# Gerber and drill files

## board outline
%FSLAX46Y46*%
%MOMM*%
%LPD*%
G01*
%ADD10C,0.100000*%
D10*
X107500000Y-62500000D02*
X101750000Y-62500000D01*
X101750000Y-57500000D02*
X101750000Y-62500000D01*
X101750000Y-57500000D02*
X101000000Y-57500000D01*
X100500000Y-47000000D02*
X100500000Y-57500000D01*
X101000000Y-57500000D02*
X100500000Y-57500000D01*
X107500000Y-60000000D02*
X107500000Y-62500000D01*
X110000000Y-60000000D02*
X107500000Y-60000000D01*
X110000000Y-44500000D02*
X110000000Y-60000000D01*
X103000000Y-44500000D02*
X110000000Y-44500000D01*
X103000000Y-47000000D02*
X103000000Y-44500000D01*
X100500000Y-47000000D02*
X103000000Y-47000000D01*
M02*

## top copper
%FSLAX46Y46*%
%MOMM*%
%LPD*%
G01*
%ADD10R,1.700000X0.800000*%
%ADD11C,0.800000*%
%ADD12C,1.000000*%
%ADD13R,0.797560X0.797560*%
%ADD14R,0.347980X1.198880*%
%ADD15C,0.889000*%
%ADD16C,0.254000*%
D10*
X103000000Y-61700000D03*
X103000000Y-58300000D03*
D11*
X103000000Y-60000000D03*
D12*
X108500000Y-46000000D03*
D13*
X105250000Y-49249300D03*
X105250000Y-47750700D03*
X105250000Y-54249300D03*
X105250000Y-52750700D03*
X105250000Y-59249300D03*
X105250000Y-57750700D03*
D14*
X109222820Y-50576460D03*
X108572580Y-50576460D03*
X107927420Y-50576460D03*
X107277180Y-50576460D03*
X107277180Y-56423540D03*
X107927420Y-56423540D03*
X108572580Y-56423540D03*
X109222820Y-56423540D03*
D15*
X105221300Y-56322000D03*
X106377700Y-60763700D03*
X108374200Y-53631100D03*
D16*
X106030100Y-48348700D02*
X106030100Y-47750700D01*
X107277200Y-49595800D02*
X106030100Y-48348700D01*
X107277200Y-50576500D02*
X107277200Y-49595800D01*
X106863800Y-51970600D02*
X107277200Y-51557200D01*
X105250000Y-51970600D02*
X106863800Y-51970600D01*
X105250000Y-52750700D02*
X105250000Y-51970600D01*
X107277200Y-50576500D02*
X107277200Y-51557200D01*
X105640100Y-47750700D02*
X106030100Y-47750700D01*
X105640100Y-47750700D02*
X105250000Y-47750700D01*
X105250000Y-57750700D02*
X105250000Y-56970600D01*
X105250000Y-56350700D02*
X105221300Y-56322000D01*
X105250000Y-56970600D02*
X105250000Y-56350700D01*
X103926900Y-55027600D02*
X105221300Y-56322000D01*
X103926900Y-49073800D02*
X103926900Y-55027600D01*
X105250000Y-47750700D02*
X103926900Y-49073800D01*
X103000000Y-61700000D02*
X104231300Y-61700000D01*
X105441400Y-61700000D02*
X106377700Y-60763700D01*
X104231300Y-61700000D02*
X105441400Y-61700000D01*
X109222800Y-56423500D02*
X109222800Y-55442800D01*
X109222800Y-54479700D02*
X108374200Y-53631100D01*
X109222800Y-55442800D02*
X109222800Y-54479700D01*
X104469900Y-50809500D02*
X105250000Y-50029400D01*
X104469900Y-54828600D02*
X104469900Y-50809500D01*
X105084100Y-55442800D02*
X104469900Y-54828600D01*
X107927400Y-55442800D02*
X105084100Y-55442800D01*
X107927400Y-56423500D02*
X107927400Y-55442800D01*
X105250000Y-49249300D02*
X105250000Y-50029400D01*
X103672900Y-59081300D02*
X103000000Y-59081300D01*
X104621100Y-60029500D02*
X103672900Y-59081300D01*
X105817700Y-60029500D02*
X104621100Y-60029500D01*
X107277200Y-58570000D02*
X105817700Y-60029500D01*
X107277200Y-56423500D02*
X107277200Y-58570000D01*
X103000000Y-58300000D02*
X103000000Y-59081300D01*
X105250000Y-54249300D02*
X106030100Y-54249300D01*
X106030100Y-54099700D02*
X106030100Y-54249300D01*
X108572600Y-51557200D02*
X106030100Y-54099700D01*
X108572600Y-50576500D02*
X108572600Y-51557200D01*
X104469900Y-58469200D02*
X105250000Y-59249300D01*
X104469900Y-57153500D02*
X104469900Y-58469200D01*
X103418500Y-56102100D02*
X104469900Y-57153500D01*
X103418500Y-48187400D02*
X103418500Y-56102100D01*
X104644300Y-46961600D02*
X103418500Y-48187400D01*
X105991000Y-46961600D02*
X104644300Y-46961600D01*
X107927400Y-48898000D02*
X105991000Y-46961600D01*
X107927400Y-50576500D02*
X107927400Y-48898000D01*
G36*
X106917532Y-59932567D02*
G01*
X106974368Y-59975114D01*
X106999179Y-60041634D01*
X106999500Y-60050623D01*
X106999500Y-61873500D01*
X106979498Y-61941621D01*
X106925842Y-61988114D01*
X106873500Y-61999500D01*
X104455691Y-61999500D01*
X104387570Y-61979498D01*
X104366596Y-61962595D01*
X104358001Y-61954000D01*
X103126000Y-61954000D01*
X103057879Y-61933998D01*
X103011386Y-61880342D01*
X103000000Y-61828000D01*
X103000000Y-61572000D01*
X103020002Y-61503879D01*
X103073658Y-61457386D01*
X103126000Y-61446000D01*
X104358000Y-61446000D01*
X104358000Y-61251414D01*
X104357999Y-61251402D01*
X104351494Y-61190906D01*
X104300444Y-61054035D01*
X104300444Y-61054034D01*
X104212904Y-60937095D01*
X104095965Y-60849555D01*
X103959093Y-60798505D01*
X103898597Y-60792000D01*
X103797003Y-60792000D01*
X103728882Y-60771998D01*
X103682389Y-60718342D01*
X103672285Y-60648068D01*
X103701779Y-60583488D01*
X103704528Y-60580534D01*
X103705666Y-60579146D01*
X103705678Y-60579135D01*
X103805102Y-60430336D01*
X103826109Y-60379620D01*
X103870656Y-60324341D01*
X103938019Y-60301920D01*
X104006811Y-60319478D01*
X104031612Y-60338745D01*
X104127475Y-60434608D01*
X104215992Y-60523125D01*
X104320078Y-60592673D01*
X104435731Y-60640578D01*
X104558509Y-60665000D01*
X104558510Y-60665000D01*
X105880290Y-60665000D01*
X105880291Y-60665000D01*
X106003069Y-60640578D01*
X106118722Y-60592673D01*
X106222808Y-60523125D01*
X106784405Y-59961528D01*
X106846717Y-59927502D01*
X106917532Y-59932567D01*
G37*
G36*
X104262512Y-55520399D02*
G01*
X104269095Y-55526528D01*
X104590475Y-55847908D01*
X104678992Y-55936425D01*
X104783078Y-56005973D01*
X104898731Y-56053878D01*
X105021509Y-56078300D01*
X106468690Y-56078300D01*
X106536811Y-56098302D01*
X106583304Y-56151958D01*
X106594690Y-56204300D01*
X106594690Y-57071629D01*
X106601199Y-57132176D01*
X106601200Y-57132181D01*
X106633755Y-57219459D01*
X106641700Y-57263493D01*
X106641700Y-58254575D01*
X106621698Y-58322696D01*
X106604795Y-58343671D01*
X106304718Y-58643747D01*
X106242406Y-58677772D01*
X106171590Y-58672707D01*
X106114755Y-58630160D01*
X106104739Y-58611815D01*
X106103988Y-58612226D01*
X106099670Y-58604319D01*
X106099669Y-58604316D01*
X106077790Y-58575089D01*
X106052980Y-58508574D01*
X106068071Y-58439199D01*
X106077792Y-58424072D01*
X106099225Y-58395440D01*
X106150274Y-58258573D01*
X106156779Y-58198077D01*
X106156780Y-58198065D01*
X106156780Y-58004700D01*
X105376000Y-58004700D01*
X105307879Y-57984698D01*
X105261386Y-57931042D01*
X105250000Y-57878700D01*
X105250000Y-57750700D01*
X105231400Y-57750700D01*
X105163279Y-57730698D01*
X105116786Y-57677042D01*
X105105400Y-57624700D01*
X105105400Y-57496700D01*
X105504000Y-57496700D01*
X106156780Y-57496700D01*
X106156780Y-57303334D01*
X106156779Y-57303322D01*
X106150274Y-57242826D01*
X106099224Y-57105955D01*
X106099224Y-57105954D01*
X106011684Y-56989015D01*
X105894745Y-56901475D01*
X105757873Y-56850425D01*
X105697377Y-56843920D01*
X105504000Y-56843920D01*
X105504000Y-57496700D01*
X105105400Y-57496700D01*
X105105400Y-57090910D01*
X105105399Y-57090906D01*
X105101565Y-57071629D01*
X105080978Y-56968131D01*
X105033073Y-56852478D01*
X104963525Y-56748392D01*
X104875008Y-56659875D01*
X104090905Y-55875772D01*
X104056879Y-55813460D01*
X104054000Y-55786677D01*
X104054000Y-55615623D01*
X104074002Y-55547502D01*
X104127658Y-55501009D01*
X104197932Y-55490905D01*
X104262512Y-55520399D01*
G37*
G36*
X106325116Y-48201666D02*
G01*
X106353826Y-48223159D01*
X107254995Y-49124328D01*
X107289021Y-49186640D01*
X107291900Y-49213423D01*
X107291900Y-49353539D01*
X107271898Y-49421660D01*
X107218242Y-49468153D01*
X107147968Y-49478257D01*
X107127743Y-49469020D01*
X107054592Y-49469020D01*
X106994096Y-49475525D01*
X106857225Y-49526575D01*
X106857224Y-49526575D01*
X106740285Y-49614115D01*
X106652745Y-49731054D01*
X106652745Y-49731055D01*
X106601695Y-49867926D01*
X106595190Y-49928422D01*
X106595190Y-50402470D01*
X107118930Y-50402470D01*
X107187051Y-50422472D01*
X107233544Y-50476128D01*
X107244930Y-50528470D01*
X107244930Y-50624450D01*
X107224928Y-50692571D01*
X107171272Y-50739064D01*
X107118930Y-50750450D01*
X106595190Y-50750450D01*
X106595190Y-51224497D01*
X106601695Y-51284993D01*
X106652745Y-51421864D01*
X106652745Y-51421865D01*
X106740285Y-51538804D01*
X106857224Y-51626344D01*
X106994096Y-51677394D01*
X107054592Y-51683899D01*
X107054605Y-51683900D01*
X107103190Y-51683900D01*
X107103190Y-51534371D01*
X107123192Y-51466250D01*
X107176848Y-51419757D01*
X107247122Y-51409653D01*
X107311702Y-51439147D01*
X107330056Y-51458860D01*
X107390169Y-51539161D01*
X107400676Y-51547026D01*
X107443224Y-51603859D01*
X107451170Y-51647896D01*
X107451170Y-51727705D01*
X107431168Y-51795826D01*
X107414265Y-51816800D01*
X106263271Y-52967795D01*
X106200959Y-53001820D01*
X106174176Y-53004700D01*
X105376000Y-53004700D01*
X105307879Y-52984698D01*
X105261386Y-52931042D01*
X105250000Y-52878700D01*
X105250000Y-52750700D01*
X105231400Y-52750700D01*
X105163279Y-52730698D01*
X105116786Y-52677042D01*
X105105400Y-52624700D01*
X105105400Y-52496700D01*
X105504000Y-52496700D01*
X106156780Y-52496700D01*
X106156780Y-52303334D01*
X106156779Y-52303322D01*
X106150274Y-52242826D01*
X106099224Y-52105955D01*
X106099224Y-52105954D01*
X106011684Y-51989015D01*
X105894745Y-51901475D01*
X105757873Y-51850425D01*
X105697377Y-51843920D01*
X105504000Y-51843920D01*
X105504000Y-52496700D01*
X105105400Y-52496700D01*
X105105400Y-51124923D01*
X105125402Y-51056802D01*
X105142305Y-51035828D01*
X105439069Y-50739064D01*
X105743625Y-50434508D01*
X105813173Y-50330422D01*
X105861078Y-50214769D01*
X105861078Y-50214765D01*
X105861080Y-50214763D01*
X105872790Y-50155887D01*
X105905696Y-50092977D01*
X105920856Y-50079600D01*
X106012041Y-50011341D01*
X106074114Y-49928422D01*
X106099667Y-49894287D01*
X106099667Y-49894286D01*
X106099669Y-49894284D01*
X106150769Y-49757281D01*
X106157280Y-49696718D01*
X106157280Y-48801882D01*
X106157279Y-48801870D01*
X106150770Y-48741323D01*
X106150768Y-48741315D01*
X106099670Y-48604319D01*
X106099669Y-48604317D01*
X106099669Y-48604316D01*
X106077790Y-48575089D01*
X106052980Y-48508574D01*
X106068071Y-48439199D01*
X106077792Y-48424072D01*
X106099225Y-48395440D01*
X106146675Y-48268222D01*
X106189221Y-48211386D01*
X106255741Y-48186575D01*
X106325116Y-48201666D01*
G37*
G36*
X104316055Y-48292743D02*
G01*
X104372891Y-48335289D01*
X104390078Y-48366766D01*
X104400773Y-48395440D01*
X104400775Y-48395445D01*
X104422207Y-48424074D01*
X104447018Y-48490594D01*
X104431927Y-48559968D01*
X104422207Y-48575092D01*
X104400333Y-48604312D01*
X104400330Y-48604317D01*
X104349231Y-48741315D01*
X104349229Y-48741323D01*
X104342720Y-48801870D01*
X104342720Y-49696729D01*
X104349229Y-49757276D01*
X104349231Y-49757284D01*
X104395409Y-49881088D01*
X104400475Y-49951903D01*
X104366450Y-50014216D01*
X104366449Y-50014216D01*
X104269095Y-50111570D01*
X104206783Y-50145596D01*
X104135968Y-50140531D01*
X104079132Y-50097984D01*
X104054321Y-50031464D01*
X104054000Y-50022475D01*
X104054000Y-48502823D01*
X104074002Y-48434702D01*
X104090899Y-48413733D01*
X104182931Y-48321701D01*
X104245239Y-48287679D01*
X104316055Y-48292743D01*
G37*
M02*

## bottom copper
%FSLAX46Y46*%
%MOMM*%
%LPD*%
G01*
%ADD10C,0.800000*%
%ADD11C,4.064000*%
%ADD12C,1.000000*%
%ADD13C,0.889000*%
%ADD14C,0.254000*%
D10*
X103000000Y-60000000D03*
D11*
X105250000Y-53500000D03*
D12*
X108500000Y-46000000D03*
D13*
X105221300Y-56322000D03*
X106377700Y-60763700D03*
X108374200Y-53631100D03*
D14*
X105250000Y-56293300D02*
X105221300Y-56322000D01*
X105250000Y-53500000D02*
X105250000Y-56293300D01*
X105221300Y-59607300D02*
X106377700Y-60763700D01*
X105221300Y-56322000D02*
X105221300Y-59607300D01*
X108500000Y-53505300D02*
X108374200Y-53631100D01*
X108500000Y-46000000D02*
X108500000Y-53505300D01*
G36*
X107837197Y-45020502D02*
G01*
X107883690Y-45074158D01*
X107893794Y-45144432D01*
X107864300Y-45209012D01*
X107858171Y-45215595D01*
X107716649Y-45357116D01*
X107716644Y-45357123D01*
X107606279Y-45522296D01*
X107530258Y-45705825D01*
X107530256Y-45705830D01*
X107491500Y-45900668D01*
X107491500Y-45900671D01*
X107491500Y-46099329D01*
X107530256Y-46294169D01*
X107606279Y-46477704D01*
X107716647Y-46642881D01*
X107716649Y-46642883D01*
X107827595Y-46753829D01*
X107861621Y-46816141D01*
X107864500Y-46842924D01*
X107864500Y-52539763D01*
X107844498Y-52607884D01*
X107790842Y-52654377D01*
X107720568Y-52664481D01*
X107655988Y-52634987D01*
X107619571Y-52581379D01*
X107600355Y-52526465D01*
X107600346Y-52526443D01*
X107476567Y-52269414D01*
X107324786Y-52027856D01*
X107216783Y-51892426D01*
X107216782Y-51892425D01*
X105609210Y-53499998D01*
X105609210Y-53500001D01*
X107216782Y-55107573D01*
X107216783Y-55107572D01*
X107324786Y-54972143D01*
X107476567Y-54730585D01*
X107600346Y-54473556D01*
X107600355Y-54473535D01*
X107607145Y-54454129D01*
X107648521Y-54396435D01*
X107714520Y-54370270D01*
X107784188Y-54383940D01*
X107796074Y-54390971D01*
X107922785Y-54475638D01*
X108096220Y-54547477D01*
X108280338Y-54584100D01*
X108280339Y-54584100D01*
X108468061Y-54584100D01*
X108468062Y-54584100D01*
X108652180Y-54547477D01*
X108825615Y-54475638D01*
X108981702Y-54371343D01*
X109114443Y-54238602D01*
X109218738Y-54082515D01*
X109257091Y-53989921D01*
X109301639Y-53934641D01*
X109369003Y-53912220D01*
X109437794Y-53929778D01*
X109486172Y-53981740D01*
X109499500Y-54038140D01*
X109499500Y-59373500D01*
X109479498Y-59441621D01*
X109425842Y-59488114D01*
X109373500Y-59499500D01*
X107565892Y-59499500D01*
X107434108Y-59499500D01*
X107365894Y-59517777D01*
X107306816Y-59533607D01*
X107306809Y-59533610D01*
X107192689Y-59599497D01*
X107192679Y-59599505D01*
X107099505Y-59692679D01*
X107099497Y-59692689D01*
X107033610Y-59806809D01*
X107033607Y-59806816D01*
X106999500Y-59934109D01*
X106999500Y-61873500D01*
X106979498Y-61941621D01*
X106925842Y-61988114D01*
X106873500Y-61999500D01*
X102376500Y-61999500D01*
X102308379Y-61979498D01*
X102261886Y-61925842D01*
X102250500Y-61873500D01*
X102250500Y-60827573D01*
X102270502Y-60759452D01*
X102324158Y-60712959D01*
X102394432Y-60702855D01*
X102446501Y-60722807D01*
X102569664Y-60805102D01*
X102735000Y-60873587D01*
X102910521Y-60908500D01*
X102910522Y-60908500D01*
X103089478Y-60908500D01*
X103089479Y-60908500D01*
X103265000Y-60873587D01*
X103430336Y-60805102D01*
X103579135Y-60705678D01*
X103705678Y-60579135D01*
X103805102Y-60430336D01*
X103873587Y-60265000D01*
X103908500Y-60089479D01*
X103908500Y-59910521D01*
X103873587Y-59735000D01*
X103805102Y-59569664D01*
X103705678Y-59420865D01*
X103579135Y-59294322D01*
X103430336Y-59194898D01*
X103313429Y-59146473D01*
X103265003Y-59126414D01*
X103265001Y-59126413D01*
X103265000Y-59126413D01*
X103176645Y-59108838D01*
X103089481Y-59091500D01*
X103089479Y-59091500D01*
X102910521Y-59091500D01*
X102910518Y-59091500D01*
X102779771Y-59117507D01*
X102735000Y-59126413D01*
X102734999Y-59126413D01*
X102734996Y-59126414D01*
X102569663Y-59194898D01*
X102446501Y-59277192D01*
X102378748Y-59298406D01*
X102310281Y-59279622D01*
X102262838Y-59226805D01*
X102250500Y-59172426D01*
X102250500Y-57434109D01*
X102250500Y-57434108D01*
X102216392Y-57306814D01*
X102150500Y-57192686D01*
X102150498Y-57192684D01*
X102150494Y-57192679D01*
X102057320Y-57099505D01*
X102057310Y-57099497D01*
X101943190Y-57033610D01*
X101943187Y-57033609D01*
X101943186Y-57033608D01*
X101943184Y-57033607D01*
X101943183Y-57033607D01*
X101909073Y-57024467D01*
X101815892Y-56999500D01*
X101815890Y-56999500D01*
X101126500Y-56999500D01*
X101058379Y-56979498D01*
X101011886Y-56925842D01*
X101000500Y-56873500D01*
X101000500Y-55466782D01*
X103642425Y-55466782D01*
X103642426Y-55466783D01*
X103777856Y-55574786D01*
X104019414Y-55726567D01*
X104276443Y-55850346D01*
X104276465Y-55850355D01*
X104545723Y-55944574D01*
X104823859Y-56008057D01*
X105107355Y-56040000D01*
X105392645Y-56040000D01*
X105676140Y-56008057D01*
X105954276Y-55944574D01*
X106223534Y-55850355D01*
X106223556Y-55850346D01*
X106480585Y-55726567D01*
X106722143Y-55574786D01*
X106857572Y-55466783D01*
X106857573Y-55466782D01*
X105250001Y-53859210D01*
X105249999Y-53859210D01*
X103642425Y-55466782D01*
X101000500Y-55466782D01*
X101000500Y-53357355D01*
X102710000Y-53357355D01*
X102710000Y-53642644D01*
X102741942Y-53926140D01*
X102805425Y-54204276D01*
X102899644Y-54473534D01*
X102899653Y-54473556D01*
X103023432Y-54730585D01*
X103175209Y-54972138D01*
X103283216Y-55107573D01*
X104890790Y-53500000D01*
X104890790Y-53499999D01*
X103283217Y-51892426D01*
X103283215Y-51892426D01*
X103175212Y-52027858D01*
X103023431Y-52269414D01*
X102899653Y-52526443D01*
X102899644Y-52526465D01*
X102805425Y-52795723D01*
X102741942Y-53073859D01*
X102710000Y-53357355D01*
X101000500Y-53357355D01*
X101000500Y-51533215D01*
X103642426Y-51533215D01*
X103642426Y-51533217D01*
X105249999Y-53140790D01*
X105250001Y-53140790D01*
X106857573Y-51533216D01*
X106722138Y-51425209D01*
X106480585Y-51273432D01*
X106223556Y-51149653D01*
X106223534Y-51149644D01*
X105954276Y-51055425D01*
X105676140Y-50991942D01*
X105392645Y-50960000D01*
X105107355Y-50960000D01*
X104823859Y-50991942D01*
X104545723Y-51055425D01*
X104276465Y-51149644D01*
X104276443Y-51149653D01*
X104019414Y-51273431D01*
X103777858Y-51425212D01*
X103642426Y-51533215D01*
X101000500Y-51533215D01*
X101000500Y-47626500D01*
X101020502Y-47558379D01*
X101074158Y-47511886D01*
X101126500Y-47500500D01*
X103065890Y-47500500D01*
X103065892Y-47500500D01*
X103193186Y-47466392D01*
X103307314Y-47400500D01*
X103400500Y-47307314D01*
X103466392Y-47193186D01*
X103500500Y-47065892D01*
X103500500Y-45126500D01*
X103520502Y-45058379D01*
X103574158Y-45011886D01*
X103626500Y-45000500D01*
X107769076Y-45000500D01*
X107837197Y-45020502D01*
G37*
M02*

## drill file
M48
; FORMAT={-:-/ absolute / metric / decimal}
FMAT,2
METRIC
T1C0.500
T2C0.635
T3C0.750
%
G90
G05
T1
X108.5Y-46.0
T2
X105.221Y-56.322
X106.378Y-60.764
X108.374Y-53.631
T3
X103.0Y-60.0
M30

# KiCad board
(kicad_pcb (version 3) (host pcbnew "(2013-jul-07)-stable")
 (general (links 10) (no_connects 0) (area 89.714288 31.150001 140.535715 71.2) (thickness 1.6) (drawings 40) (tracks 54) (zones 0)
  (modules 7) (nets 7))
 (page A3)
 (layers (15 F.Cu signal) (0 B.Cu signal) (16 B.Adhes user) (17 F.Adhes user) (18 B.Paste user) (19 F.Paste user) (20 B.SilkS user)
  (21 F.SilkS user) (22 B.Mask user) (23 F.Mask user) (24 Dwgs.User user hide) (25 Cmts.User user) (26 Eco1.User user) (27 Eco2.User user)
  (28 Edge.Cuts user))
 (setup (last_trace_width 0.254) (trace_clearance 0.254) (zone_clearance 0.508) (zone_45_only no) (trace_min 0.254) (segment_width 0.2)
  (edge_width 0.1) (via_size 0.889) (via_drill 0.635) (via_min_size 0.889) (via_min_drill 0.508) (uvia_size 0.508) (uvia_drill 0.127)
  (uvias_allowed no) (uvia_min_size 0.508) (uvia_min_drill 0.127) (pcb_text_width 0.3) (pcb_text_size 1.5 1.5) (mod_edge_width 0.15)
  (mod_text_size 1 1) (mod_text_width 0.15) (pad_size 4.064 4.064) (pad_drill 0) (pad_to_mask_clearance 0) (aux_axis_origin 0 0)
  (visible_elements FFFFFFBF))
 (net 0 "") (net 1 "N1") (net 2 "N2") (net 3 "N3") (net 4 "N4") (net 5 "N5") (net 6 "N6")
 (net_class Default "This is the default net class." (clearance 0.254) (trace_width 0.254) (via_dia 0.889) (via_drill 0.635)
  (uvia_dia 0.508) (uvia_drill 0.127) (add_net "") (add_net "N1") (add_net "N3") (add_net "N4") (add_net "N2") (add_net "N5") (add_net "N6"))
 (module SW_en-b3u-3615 (layer F.Cu) (at 103 60 90)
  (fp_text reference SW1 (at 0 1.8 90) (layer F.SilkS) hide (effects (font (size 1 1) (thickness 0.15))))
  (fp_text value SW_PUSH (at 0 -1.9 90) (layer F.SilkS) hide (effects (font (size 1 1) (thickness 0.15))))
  (pad 1 smd rect (at -1.7 0 90) (size 0.8 1.7) (layers F.Cu F.Paste F.Mask) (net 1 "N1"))
  (pad 2 smd rect (at 1.7 0 90) (size 0.8 1.7) (layers F.Cu F.Paste F.Mask) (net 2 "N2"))
  (pad "" thru_hole circle (at 0 0 90) (size 0.8 0.8) (drill 0.75) (layers *.Cu *.Mask F.SilkS)))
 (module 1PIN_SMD (layer B.Cu) (at 105.25 53.5)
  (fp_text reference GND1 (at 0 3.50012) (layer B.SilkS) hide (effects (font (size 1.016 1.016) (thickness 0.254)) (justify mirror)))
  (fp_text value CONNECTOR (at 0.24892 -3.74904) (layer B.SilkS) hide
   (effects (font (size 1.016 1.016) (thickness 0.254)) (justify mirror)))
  (pad 1 smd circle (at 0 0) (size 4.064 4.064) (layers B.Cu B.Paste B.Mask) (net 1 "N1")))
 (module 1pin (layer F.Cu) (at 108.5 46)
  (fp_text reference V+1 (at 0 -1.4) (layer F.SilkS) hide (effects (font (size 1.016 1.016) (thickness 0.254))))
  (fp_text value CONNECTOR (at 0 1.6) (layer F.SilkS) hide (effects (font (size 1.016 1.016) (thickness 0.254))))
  (pad 1 thru_hole circle (at 0 0) (size 1 1) (drill 0.5) (layers *.Cu *.Mask F.SilkS) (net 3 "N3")))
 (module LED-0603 (layer F.Cu) (at 105.25 48.5 90)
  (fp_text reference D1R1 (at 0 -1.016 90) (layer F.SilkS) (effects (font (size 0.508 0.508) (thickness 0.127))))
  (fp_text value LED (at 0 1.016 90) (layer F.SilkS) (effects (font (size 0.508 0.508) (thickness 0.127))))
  (pad 1 smd rect (at -0.7493 0 90) (size 0.79756 0.79756) (layers F.Cu F.Paste F.Mask) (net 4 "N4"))
  (pad 2 smd rect (at 0.7493 0 90) (size 0.79756 0.79756) (layers F.Cu F.Paste F.Mask) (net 1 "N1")))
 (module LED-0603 (layer F.Cu) (at 105.25 53.5 90)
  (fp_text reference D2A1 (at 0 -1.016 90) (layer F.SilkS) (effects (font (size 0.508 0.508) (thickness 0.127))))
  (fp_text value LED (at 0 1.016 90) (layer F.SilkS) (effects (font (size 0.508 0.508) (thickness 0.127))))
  (pad 1 smd rect (at -0.7493 0 90) (size 0.79756 0.79756) (layers F.Cu F.Paste F.Mask) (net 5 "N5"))
  (pad 2 smd rect (at 0.7493 0 90) (size 0.79756 0.79756) (layers F.Cu F.Paste F.Mask) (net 1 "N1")))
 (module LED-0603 (layer F.Cu) (at 105.25 58.5 90)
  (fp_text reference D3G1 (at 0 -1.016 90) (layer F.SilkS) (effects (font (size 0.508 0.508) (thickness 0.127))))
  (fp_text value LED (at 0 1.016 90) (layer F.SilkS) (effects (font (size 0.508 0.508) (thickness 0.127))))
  (pad 1 smd rect (at -0.7493 0 90) (size 0.79756 0.79756) (layers F.Cu F.Paste F.Mask) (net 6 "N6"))
  (pad 2 smd rect (at 0.7493 0 90) (size 0.79756 0.79756) (layers F.Cu F.Paste F.Mask) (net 1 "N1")))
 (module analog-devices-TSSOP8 (layer F.Cu) (at 108.25 53.5 270)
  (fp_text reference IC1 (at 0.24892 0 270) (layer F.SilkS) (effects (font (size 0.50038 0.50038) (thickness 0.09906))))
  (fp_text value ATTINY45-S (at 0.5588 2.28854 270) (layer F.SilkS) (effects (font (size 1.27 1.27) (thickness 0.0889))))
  (pad 1 smd rect (at -2.92354 -0.97282 270) (size 1.19888 0.34798) (layers F.Cu F.Paste F.Mask))
  (pad 2 smd rect (at -2.92354 -0.32258 270) (size 1.19888 0.34798) (layers F.Cu F.Paste F.Mask) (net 5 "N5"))
  (pad 3 smd rect (at -2.92354 0.32258 270) (size 1.19888 0.34798) (layers F.Cu F.Paste F.Mask) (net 6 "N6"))
  (pad 4 smd rect (at -2.92354 0.97282 270) (size 1.19888 0.34798) (layers F.Cu F.Paste F.Mask) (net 1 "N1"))
  (pad 5 smd rect (at 2.92354 0.97282 270) (size 1.19888 0.34798) (layers F.Cu F.Paste F.Mask) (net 2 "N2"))
  (pad 6 smd rect (at 2.92354 0.32258 270) (size 1.19888 0.34798) (layers F.Cu F.Paste F.Mask) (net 4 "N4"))
  (pad 7 smd rect (at 2.92354 -0.32258 270) (size 1.19888 0.34798) (layers F.Cu F.Paste F.Mask))
  (pad 8 smd rect (at 2.92354 -0.97282 270) (size 1.19888 0.34798) (layers F.Cu F.Paste F.Mask) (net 3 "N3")))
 (gr_line (start 107.5 62.5) (end 101.75 62.5) (angle 90) (layer Edge.Cuts) (width 0.1))
 (gr_line (start 101.75 57.5) (end 101.75 62.5) (angle 90) (layer Edge.Cuts) (width 0.1))
 (gr_line (start 101.75 57.5) (end 101 57.5) (angle 90) (layer Edge.Cuts) (width 0.1))
 (gr_line (start 100.5 47) (end 100.5 57.5) (angle 90) (layer Edge.Cuts) (width 0.1))
 (gr_line (start 101 57.5) (end 100.5 57.5) (angle 90) (layer Edge.Cuts) (width 0.1))
 (gr_line (start 107.5 60) (end 107.5 62.5) (angle 90) (layer Edge.Cuts) (width 0.1))
 (gr_line (start 110 60) (end 107.5 60) (angle 90) (layer Edge.Cuts) (width 0.1))
 (gr_line (start 110 44.5) (end 110 60) (angle 90) (layer Edge.Cuts) (width 0.1))
 (gr_line (start 103 44.5) (end 110 44.5) (angle 90) (layer Edge.Cuts) (width 0.1))
 (gr_line (start 103 47) (end 103 44.5) (angle 90) (layer Edge.Cuts) (width 0.1))
 (gr_line (start 100.5 47) (end 103 47) (angle 90) (layer Edge.Cuts) (width 0.1))
 (via (at 105.2213 56.322) (size 0.889) (layers F.Cu B.Cu) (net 1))
 (via (at 106.3777 60.7637) (size 0.889) (layers F.Cu B.Cu) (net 1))
 (segment (start 106.0301 48.3487) (end 106.0301 47.7507) (width 0.254) (layer F.Cu) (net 1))
 (segment (start 107.2772 49.5958) (end 106.0301 48.3487) (width 0.254) (layer F.Cu) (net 1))
 (segment (start 107.2772 50.5765) (end 107.2772 49.5958) (width 0.254) (layer F.Cu) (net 1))
 (segment (start 106.8638 51.9706) (end 107.2772 51.5572) (width 0.254) (layer F.Cu) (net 1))
 (segment (start 105.25 51.9706) (end 106.8638 51.9706) (width 0.254) (layer F.Cu) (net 1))
 (segment (start 105.25 52.7507) (end 105.25 51.9706) (width 0.254) (layer F.Cu) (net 1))
 (segment (start 107.2772 50.5765) (end 107.2772 51.5572) (width 0.254) (layer F.Cu) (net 1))
 (segment (start 105.6401 47.7507) (end 106.0301 47.7507) (width 0.254) (layer F.Cu) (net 1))
 (segment (start 105.6401 47.7507) (end 105.25 47.7507) (width 0.254) (layer F.Cu) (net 1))
 (segment (start 105.25 57.7507) (end 105.25 56.9706) (width 0.254) (layer F.Cu) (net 1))
 (segment (start 105.25 56.3507) (end 105.2213 56.322) (width 0.254) (layer F.Cu) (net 1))
 (segment (start 105.25 56.9706) (end 105.25 56.3507) (width 0.254) (layer F.Cu) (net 1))
 (segment (start 103.9269 55.0276) (end 105.2213 56.322) (width 0.254) (layer F.Cu) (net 1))
 (segment (start 103.9269 49.0738) (end 103.9269 55.0276) (width 0.254) (layer F.Cu) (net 1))
 (segment (start 105.25 47.7507) (end 103.9269 49.0738) (width 0.254) (layer F.Cu) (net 1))
 (segment (start 103 61.7) (end 104.2313 61.7) (width 0.254) (layer F.Cu) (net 1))
 (segment (start 105.25 56.2933) (end 105.2213 56.322) (width 0.254) (layer B.Cu) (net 1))
 (segment (start 105.25 53.5) (end 105.25 56.2933) (width 0.254) (layer B.Cu) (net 1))
 (segment (start 105.2213 59.6073) (end 106.3777 60.7637) (width 0.254) (layer B.Cu) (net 1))
 (segment (start 105.2213 56.322) (end 105.2213 59.6073) (width 0.254) (layer B.Cu) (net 1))
 (segment (start 105.4414 61.7) (end 106.3777 60.7637) (width 0.254) (layer F.Cu) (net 1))
 (segment (start 104.2313 61.7) (end 105.4414 61.7) (width 0.254) (layer F.Cu) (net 1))
 (via (at 108.3742 53.6311) (size 0.889) (layers F.Cu B.Cu) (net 3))
 (segment (start 109.2228 56.4235) (end 109.2228 55.4428) (width 0.254) (layer F.Cu) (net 3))
 (segment (start 108.5 53.5053) (end 108.3742 53.6311) (width 0.254) (layer B.Cu) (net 3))
 (segment (start 108.5 46) (end 108.5 53.5053) (width 0.254) (layer B.Cu) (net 3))
 (segment (start 109.2228 54.4797) (end 108.3742 53.6311) (width 0.254) (layer F.Cu) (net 3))
 (segment (start 109.2228 55.4428) (end 109.2228 54.4797) (width 0.254) (layer F.Cu) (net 3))
 (segment (start 104.4699 50.8095) (end 105.25 50.0294) (width 0.254) (layer F.Cu) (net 4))
 (segment (start 104.4699 54.8286) (end 104.4699 50.8095) (width 0.254) (layer F.Cu) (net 4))
 (segment (start 105.0841 55.4428) (end 104.4699 54.8286) (width 0.254) (layer F.Cu) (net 4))
 (segment (start 107.9274 55.4428) (end 105.0841 55.4428) (width 0.254) (layer F.Cu) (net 4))
 (segment (start 107.9274 56.4235) (end 107.9274 55.4428) (width 0.254) (layer F.Cu) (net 4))
 (segment (start 105.25 49.2493) (end 105.25 50.0294) (width 0.254) (layer F.Cu) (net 4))
 (segment (start 103.6729 59.0813) (end 103 59.0813) (width 0.254) (layer F.Cu) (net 2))
 (segment (start 104.6211 60.0295) (end 103.6729 59.0813) (width 0.254) (layer F.Cu) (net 2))
 (segment (start 105.8177 60.0295) (end 104.6211 60.0295) (width 0.254) (layer F.Cu) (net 2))
 (segment (start 107.2772 58.57) (end 105.8177 60.0295) (width 0.254) (layer F.Cu) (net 2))
 (segment (start 107.2772 56.4235) (end 107.2772 58.57) (width 0.254) (layer F.Cu) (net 2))
 (segment (start 103 58.3) (end 103 59.0813) (width 0.254) (layer F.Cu) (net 2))
 (segment (start 105.25 54.2493) (end 106.0301 54.2493) (width 0.254) (layer F.Cu) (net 5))
 (segment (start 106.0301 54.0997) (end 106.0301 54.2493) (width 0.254) (layer F.Cu) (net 5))
 (segment (start 108.5726 51.5572) (end 106.0301 54.0997) (width 0.254) (layer F.Cu) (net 5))
 (segment (start 108.5726 50.5765) (end 108.5726 51.5572) (width 0.254) (layer F.Cu) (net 5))
 (segment (start 104.4699 58.4692) (end 105.25 59.2493) (width 0.254) (layer F.Cu) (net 6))
 (segment (start 104.4699 57.1535) (end 104.4699 58.4692) (width 0.254) (layer F.Cu) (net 6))
 (segment (start 103.4185 56.1021) (end 104.4699 57.1535) (width 0.254) (layer F.Cu) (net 6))
 (segment (start 103.4185 48.1874) (end 103.4185 56.1021) (width 0.254) (layer F.Cu) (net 6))
 (segment (start 104.6443 46.9616) (end 103.4185 48.1874) (width 0.254) (layer F.Cu) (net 6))
 (segment (start 105.991 46.9616) (end 104.6443 46.9616) (width 0.254) (layer F.Cu) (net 6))
 (segment (start 107.9274 48.898) (end 105.991 46.9616) (width 0.254) (layer F.Cu) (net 6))
 (segment (start 107.9274 50.5765) (end 107.9274 48.898) (width 0.254) (layer F.Cu) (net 6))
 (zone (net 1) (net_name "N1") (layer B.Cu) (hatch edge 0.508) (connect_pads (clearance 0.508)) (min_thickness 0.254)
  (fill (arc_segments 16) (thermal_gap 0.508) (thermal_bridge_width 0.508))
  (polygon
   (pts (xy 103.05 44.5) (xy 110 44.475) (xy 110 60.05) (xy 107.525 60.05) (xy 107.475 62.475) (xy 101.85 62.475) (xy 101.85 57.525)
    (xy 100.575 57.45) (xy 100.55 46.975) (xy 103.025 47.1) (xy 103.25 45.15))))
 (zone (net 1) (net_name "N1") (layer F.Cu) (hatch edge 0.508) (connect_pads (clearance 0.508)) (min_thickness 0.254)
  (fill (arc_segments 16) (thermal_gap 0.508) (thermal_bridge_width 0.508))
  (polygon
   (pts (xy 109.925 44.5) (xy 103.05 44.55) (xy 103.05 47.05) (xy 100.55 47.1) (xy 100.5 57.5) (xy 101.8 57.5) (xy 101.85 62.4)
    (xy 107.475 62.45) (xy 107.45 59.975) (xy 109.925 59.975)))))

